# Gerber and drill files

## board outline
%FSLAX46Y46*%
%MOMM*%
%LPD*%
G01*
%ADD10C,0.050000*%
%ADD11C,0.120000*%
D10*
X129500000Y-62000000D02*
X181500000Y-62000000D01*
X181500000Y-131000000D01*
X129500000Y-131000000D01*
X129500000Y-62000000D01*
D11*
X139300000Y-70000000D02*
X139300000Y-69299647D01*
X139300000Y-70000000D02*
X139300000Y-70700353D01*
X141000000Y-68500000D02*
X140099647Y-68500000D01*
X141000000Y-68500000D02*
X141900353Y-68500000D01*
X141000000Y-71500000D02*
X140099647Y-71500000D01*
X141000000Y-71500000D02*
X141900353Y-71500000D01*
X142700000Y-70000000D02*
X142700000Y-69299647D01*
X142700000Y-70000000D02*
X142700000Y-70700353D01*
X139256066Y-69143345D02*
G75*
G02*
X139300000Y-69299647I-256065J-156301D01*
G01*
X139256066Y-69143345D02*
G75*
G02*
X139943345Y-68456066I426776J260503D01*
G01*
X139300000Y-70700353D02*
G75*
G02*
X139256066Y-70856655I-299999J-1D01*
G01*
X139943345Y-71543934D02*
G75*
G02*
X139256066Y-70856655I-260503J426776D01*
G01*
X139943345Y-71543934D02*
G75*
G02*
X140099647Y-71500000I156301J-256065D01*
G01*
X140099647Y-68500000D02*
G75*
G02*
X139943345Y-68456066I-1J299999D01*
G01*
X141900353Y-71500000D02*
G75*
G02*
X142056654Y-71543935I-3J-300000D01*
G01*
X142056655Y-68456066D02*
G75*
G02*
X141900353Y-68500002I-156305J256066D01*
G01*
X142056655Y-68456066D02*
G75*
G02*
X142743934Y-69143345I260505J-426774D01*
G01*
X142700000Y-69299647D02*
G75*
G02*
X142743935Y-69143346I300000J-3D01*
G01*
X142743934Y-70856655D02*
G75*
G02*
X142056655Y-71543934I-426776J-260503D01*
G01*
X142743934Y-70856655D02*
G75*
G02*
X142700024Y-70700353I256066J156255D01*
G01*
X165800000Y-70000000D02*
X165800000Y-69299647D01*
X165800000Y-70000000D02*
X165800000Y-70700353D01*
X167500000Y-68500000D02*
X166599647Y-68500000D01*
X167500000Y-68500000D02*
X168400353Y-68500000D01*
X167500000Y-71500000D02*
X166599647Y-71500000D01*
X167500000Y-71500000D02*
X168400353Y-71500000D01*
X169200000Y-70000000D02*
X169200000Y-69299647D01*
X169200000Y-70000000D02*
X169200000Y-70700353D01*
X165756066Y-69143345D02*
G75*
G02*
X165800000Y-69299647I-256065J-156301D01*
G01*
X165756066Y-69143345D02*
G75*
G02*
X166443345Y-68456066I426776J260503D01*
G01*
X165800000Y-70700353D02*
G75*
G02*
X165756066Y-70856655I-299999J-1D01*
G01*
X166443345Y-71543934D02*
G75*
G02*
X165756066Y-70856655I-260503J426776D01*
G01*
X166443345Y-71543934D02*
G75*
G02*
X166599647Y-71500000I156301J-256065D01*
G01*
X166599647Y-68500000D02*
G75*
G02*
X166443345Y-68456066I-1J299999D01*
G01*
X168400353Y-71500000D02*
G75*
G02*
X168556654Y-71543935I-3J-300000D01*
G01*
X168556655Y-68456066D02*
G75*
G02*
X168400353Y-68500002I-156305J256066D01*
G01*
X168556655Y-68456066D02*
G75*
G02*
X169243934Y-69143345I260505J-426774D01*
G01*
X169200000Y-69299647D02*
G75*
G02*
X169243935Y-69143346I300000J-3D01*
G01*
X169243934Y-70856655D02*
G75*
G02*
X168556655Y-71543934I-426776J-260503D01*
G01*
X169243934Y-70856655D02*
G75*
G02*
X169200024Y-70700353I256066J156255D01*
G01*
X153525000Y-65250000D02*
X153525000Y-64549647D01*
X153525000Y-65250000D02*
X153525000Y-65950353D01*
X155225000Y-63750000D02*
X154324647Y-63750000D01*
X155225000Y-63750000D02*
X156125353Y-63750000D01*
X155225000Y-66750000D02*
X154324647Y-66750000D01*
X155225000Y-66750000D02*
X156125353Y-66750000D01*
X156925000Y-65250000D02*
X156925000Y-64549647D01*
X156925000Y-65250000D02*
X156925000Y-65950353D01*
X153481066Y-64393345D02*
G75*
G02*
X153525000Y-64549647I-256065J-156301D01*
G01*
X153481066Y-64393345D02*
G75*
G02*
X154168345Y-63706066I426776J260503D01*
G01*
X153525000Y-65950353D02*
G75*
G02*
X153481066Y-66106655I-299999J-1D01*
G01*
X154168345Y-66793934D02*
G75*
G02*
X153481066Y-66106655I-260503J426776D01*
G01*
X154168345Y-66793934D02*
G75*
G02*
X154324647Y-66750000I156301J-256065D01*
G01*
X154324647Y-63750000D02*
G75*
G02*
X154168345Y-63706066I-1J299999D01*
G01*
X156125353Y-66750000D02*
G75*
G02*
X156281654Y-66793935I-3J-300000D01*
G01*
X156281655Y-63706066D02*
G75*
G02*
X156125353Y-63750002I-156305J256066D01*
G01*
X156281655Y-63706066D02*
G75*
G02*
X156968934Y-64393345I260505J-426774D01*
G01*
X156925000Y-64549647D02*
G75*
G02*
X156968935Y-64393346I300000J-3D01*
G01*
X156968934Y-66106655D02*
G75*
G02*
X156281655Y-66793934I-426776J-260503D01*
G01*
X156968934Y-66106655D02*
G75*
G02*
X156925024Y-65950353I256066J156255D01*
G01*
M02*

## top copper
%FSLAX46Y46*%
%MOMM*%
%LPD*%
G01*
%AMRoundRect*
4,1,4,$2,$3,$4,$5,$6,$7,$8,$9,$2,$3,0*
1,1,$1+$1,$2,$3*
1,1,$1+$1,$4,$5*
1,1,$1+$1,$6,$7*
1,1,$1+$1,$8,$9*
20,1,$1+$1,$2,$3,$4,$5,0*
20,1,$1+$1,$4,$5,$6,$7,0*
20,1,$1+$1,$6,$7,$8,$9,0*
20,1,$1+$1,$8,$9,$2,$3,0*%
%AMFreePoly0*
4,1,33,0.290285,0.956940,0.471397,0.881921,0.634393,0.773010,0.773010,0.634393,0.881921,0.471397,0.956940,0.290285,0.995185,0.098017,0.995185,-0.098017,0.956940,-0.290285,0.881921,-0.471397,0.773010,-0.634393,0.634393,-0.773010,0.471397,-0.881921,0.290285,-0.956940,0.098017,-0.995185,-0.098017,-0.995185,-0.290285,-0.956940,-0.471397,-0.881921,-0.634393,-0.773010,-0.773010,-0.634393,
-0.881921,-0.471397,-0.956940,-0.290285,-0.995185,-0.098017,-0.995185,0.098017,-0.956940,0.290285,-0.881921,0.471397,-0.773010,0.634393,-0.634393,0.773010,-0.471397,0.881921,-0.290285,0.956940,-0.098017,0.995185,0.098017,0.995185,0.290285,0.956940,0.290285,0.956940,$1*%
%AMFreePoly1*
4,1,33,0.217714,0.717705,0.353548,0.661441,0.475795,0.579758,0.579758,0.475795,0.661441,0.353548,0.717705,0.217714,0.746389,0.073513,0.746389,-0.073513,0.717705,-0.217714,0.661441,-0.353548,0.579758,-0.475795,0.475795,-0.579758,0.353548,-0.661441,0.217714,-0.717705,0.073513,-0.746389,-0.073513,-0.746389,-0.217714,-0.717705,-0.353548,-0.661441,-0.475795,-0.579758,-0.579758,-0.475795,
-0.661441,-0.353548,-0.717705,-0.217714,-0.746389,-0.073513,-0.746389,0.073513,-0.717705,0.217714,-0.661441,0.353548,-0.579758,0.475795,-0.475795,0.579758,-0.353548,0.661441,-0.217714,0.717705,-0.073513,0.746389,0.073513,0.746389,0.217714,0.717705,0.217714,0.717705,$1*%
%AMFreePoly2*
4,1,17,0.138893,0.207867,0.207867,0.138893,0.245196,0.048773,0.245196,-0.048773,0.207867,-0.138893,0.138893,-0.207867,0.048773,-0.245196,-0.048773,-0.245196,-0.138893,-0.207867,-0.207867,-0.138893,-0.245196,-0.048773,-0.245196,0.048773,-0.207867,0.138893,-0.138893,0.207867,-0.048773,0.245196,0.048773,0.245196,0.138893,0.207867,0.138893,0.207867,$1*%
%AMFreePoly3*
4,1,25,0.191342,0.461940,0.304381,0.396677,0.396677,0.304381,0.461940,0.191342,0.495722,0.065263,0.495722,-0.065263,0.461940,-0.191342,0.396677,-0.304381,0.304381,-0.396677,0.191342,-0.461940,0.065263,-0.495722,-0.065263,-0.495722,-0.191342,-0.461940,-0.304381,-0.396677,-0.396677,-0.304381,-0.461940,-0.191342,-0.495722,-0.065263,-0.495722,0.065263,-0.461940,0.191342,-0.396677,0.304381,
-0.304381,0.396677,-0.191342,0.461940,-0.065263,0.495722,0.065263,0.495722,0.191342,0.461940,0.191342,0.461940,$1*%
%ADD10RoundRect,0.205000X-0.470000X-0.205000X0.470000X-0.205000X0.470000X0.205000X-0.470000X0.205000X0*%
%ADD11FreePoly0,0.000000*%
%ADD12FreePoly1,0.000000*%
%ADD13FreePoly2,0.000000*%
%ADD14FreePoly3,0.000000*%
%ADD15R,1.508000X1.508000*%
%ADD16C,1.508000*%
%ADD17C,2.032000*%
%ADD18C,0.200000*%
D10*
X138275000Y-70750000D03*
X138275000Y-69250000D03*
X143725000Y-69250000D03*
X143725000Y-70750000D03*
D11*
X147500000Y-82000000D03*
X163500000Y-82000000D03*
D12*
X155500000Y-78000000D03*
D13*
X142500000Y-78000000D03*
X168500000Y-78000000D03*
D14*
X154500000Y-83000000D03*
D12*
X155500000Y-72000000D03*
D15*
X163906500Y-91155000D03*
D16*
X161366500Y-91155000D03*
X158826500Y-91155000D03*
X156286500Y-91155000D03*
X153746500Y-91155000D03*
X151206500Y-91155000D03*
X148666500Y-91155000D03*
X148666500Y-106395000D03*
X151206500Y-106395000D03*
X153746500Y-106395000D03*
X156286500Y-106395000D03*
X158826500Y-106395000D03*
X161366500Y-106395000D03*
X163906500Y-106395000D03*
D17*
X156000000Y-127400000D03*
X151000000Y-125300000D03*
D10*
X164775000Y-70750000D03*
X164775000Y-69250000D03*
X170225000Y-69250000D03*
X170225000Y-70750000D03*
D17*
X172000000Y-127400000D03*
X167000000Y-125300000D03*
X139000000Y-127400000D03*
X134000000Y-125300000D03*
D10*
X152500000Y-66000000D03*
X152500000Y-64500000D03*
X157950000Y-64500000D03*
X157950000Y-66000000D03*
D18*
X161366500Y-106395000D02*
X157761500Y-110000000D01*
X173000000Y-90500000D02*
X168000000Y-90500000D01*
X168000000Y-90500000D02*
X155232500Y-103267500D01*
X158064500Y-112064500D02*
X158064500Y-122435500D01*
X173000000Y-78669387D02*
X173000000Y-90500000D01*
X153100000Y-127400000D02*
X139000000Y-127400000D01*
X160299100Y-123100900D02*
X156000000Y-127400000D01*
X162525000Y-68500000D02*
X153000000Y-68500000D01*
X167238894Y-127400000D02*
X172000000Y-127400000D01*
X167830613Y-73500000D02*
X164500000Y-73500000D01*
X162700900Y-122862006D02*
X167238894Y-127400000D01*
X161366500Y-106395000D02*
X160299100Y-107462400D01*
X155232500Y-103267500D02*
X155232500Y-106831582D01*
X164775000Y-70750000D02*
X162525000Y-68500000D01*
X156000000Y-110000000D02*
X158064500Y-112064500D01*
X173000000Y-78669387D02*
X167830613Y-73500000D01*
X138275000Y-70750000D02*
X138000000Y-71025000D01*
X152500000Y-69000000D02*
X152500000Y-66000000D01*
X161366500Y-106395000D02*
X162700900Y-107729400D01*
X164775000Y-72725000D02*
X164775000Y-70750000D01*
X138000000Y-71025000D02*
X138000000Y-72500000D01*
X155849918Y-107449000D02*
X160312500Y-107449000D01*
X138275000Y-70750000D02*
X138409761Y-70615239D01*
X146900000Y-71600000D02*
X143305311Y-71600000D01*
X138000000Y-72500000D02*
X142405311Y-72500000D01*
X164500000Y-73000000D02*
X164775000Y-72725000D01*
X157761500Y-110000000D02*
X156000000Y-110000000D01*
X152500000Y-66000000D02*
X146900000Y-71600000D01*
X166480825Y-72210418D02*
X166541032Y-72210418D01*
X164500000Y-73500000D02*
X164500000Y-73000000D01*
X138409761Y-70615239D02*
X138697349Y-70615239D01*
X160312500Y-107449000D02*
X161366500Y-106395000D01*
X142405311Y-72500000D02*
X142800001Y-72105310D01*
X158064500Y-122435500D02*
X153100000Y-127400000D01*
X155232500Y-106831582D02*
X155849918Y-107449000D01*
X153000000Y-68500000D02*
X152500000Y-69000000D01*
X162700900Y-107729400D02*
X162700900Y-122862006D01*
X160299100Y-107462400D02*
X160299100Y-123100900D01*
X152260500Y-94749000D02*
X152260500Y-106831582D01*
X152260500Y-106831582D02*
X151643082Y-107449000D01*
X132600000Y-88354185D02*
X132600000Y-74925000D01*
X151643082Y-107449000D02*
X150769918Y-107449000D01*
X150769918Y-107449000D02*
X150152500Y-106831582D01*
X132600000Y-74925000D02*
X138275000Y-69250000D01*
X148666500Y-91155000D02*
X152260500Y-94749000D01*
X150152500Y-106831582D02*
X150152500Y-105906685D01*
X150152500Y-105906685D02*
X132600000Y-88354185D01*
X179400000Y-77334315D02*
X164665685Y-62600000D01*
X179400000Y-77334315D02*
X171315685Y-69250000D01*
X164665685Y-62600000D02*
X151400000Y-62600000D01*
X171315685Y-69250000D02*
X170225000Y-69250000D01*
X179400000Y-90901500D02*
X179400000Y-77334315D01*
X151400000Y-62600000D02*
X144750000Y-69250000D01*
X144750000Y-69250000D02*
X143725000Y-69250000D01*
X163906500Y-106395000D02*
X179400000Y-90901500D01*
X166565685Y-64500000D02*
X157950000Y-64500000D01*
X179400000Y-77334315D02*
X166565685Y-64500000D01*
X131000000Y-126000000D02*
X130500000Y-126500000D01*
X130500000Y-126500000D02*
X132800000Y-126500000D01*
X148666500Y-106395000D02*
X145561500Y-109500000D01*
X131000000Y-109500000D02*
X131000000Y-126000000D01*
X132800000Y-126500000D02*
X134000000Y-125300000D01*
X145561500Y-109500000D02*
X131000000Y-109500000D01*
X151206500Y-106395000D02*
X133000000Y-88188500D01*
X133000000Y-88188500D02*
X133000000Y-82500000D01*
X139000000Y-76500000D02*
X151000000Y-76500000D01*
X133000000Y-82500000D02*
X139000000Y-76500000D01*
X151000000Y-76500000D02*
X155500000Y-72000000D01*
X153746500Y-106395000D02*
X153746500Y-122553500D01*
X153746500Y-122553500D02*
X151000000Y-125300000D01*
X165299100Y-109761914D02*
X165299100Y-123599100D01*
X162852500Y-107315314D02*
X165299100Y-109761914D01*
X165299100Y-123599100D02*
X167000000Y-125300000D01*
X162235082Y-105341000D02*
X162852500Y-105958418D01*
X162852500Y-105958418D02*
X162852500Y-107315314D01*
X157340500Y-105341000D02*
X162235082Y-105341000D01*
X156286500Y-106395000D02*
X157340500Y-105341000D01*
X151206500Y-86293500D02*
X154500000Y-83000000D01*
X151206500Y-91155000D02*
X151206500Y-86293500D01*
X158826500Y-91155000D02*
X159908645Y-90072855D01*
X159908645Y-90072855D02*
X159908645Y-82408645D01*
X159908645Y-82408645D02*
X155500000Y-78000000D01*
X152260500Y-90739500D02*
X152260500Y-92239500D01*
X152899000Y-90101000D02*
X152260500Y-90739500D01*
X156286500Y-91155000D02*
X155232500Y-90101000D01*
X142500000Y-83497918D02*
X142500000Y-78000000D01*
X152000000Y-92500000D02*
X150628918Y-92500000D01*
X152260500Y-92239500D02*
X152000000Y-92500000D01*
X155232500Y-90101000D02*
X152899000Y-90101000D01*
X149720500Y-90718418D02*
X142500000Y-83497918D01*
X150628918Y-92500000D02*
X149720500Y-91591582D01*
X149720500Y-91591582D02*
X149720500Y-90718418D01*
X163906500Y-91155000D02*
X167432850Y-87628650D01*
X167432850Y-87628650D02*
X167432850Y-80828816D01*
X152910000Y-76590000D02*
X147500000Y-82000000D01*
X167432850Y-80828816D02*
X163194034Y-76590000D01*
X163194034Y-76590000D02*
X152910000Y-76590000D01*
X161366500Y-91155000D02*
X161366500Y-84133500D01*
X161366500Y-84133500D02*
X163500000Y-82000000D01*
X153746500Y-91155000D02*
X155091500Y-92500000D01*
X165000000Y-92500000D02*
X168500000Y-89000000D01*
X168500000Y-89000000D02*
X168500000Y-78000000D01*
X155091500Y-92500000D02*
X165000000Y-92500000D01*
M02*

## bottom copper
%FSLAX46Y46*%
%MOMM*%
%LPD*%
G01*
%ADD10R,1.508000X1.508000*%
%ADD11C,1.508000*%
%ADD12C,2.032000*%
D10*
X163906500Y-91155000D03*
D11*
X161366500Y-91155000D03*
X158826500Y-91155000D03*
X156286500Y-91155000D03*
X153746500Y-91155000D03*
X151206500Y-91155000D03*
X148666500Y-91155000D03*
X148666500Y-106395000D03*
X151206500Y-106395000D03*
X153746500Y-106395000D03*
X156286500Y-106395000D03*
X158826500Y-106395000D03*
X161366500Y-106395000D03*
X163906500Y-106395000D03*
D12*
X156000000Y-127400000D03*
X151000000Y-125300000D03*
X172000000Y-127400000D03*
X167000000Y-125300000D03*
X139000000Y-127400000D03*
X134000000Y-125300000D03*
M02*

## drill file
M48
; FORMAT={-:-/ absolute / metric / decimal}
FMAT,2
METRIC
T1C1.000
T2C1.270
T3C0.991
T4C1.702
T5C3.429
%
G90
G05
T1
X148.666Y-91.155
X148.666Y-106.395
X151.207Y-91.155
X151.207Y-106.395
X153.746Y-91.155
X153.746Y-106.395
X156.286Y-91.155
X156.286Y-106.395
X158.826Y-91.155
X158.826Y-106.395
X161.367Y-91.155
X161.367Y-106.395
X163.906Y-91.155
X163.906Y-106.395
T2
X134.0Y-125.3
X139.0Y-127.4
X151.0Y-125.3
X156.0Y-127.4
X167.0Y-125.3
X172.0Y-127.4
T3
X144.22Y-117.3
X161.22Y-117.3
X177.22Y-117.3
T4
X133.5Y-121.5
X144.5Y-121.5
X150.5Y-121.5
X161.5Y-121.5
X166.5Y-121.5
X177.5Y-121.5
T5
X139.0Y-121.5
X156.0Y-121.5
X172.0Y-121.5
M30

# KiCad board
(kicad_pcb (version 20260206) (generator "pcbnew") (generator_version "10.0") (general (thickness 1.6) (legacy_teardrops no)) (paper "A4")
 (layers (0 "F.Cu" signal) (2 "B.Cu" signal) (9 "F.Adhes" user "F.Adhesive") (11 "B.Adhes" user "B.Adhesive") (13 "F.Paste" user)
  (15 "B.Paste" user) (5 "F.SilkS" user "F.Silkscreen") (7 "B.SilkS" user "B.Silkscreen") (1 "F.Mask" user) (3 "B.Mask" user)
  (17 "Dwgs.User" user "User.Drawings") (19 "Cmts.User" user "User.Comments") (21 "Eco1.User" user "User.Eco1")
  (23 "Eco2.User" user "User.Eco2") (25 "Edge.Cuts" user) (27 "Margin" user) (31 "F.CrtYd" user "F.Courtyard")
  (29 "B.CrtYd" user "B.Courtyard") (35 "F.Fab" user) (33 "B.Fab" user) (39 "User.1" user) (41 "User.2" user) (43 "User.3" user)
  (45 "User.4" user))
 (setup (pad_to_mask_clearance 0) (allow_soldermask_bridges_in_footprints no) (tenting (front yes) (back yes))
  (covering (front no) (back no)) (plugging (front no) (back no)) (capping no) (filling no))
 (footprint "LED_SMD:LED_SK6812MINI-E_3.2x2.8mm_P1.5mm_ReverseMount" (layer "F.Cu") (at 141 70)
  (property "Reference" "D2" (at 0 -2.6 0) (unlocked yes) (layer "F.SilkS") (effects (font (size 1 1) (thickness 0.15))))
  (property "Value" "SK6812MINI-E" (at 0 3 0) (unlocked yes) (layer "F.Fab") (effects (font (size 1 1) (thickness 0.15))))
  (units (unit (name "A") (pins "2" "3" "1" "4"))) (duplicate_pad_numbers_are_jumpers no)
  (fp_line (start -1.7 0) (end -1.7 -0.700353) (stroke (width 0.12) (type solid)) (layer "Edge.Cuts"))
  (fp_line (start -1.7 0) (end -1.7 0.700353) (stroke (width 0.12) (type solid)) (layer "Edge.Cuts"))
  (fp_line (start 0 -1.5) (end -0.900353 -1.5) (stroke (width 0.12) (type solid)) (layer "Edge.Cuts"))
  (fp_line (start 0 -1.5) (end 0.900353 -1.5) (stroke (width 0.12) (type solid)) (layer "Edge.Cuts"))
  (fp_line (start 0 1.5) (end -0.900353 1.5) (stroke (width 0.12) (type solid)) (layer "Edge.Cuts"))
  (fp_line (start 0 1.5) (end 0.900353 1.5) (stroke (width 0.12) (type solid)) (layer "Edge.Cuts"))
  (fp_line (start 1.7 0) (end 1.7 -0.700353) (stroke (width 0.12) (type solid)) (layer "Edge.Cuts"))
  (fp_line (start 1.7 0) (end 1.7 0.700353) (stroke (width 0.12) (type solid)) (layer "Edge.Cuts"))
  (fp_arc (start -1.743934 -0.856655) (mid -1.711192 -0.781532) (end -1.7 -0.700353) (stroke (width 0.12) (type solid)) (layer "Edge.Cuts"))
  (fp_arc (start -1.743934 -0.856655) (mid -1.670711 -1.470711) (end -1.056655 -1.543934) (stroke (width 0.12) (type solid))
   (layer "Edge.Cuts"))
  (fp_arc (start -1.7 0.700353) (mid -1.711192 0.781532) (end -1.743934 0.856655) (stroke (width 0.12) (type solid)) (layer "Edge.Cuts"))
  (fp_arc (start -1.056655 1.543934) (mid -1.670711 1.470711) (end -1.743934 0.856655) (stroke (width 0.12) (type solid))
   (layer "Edge.Cuts"))
  (fp_arc (start -1.056655 1.543934) (mid -0.981532 1.511192) (end -0.900353 1.5) (stroke (width 0.12) (type solid)) (layer "Edge.Cuts"))
  (fp_arc (start -0.900353 -1.5) (mid -0.981532 -1.511192) (end -1.056655 -1.543934) (stroke (width 0.12) (type solid)) (layer "Edge.Cuts"))
  (fp_arc (start 0.900353 1.5) (mid 0.981532 1.511192) (end 1.056655 1.543934) (stroke (width 0.12) (type solid)) (layer "Edge.Cuts"))
  (fp_arc (start 1.056655 -1.543934) (mid 0.981532 -1.511192) (end 0.900353 -1.5) (stroke (width 0.12) (type solid)) (layer "Edge.Cuts"))
  (fp_arc (start 1.056655 -1.543934) (mid 1.670711 -1.470711) (end 1.743934 -0.856655) (stroke (width 0.12) (type solid))
   (layer "Edge.Cuts"))
  (fp_arc (start 1.7 -0.700353) (mid 1.711192 -0.781532) (end 1.743934 -0.856655) (stroke (width 0.12) (type solid)) (layer "Edge.Cuts"))
  (fp_arc (start 1.743934 0.856655) (mid 1.670711 1.470711) (end 1.056655 1.543934) (stroke (width 0.12) (type solid)) (layer "Edge.Cuts"))
  (fp_arc (start 1.743934 0.856655) (mid 1.711192 0.781532) (end 1.7 0.700353) (stroke (width 0.12) (type solid)) (layer "Edge.Cuts"))
  (pad "1" smd roundrect (at -2.725 0.75) (size 1.35 0.82) (layers "F.Cu" "F.Mask" "F.Paste") (roundrect_rratio 0.25) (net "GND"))
  (pad "2" smd roundrect (at -2.725 -0.75) (size 1.35 0.82) (layers "F.Cu" "F.Mask" "F.Paste") (roundrect_rratio 0.25) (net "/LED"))
  (pad "3" smd roundrect (at 2.725 -0.75) (size 1.35 0.82) (layers "F.Cu" "F.Mask" "F.Paste") (roundrect_rratio 0.25) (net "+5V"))
  (pad "4" smd roundrect (at 2.725 0.75) (size 1.35 0.82) (layers "F.Cu" "F.Mask" "F.Paste") (roundrect_rratio 0.25) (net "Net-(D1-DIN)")))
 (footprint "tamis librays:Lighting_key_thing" (layer "F.Cu") (at 149.5 71)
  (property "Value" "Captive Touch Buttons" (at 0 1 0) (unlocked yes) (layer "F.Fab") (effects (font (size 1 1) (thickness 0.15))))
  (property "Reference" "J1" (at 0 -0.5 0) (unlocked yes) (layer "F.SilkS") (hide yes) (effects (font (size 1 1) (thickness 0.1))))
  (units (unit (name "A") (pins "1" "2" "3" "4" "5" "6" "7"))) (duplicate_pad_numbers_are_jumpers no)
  (pad "1" smd custom (at -2 11) (size 2 2) (layers "F.Cu" "F.Mask") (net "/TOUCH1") (thermal_bridge_angle 90)
   (options (clearance outline) (anchor circle)) (primitives))
  (pad "2" smd custom (at 14 11) (size 2 2) (layers "F.Cu" "F.Mask") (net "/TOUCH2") (thermal_bridge_angle 90)
   (options (clearance outline) (anchor circle)) (primitives))
  (pad "3" smd custom (at 6 7) (size 1.5 5) (layers "F.Cu" "F.Mask") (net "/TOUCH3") (thermal_bridge_angle 90)
   (options (clearance outline) (anchor circle)) (primitives))
  (pad "4" smd custom (at -7 7) (size 0.5 0.5) (layers "F.Cu" "F.Mask") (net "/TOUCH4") (thermal_bridge_angle 90)
   (options (clearance outline) (anchor circle)) (primitives))
  (pad "5" smd custom (at 19 7) (size 0.5 0.5) (layers "F.Cu" "F.Mask") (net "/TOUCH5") (thermal_bridge_angle 90)
   (options (clearance outline) (anchor circle)) (primitives))
  (pad "6" smd custom (at 5 12) (size 1 1) (layers "F.Cu" "F.Mask") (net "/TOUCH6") (thermal_bridge_angle 90)
   (options (clearance outline) (anchor circle)) (primitives))
  (pad "7" smd custom (at 6 1) (size 1.5 1.5) (layers "F.Cu" "F.Mask") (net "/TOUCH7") (thermal_bridge_angle 90)
   (options (clearance outline) (anchor circle)) (primitives)))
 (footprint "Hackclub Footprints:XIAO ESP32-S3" (layer "F.Cu") (at 156.35 98.775 -90)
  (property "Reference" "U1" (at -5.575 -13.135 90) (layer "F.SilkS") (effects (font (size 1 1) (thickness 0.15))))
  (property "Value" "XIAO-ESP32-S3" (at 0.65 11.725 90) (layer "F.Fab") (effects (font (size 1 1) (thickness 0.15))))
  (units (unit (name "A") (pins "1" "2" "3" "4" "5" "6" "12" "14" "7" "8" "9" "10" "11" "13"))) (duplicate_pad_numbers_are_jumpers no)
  (pad "1" thru_hole rect (at -7.62 -7.5565 270) (size 1.508 1.508) (drill 1) (layers "*.Cu" "*.Mask") (remove_unused_layers no)
   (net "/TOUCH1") (solder_mask_margin 0.102))
  (pad "2" thru_hole circle (at -7.62 -5.0165 270) (size 1.508 1.508) (drill 1) (layers "*.Cu" "*.Mask") (remove_unused_layers no)
   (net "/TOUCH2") (solder_mask_margin 0.102))
  (pad "3" thru_hole circle (at -7.62 -2.4765 270) (size 1.508 1.508) (drill 1) (layers "*.Cu" "*.Mask") (remove_unused_layers no)
   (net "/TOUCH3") (solder_mask_margin 0.102))
  (pad "4" thru_hole circle (at -7.62 0.0635 270) (size 1.508 1.508) (drill 1) (layers "*.Cu" "*.Mask") (remove_unused_layers no)
   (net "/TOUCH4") (solder_mask_margin 0.102))
  (pad "5" thru_hole circle (at -7.62 2.6035 270) (size 1.508 1.508) (drill 1) (layers "*.Cu" "*.Mask") (remove_unused_layers no)
   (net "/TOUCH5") (solder_mask_margin 0.102))
  (pad "6" thru_hole circle (at -7.62 5.1435 270) (size 1.508 1.508) (drill 1) (layers "*.Cu" "*.Mask") (remove_unused_layers no)
   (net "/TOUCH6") (solder_mask_margin 0.102))
  (pad "7" thru_hole circle (at -7.62 7.6835 270) (size 1.508 1.508) (drill 1) (layers "*.Cu" "*.Mask") (remove_unused_layers no)
   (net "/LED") (solder_mask_margin 0.102))
  (pad "8" thru_hole circle (at 7.62 7.6835 270) (size 1.508 1.508) (drill 1) (layers "*.Cu" "*.Mask") (remove_unused_layers no)
   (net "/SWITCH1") (solder_mask_margin 0.102))
  (pad "9" thru_hole circle (at 7.62 5.1435 270) (size 1.508 1.508) (drill 1) (layers "*.Cu" "*.Mask") (remove_unused_layers no)
   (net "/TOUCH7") (solder_mask_margin 0.102))
  (pad "10" thru_hole circle (at 7.62 2.6035 270) (size 1.508 1.508) (drill 1) (layers "*.Cu" "*.Mask") (remove_unused_layers no)
   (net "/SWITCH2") (solder_mask_margin 0.102))
  (pad "11" thru_hole circle (at 7.62 0.0635 270) (size 1.508 1.508) (drill 1) (layers "*.Cu" "*.Mask") (remove_unused_layers no)
   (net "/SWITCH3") (solder_mask_margin 0.102))
  (pad "12" thru_hole circle (at 7.62 -2.4765 270) (size 1.508 1.508) (drill 1) (layers "*.Cu" "*.Mask") (remove_unused_layers no)
   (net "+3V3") (solder_mask_margin 0.102))
  (pad "13" thru_hole circle (at 7.62 -5.0165 270) (size 1.508 1.508) (drill 1) (layers "*.Cu" "*.Mask") (remove_unused_layers no)
   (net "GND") (solder_mask_margin 0.102))
  (pad "14" thru_hole circle (at 7.62 -7.5565 270) (size 1.508 1.508) (drill 1) (layers "*.Cu" "*.Mask") (remove_unused_layers no)
   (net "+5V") (solder_mask_margin 0.102)))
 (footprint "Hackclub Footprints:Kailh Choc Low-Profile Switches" (layer "F.Cu") (at 156 121.5)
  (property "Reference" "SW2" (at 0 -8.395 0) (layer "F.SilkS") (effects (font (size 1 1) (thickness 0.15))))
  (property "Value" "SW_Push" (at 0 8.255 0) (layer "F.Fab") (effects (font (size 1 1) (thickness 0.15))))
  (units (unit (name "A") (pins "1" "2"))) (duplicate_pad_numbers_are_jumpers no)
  (pad "" np_thru_hole circle (at -5.5 0) (size 1.7018 1.7018) (drill 1.7018) (layers "*.Cu" "*.Mask"))
  (pad "" np_thru_hole circle (at 0 0) (size 3.429 3.429) (drill 3.429) (layers "*.Cu" "*.Mask"))
  (pad "" np_thru_hole circle (at 5.22 -4.2) (size 0.9906 0.9906) (drill 0.9906) (layers "*.Cu" "*.Mask"))
  (pad "" np_thru_hole circle (at 5.5 0) (size 1.7018 1.7018) (drill 1.7018) (layers "*.Cu" "*.Mask"))
  (pad "1" thru_hole circle (at 0 5.9) (size 2.032 2.032) (drill 1.27) (layers "*.Cu" "*.Mask") (remove_unused_layers no) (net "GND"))
  (pad "2" thru_hole circle (at -5 3.8) (size 2.032 2.032) (drill 1.27) (layers "*.Cu" "*.Mask") (remove_unused_layers no) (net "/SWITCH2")))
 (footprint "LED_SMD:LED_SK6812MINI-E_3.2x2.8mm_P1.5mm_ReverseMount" (layer "F.Cu") (at 167.5 70)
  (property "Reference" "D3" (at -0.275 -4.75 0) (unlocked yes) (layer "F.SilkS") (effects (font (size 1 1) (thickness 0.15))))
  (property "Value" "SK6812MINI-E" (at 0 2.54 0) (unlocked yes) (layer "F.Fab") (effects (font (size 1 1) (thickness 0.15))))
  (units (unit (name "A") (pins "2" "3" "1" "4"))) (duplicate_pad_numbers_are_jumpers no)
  (fp_line (start -1.7 0) (end -1.7 -0.700353) (stroke (width 0.12) (type solid)) (layer "Edge.Cuts"))
  (fp_line (start -1.7 0) (end -1.7 0.700353) (stroke (width 0.12) (type solid)) (layer "Edge.Cuts"))
  (fp_line (start 0 -1.5) (end -0.900353 -1.5) (stroke (width 0.12) (type solid)) (layer "Edge.Cuts"))
  (fp_line (start 0 -1.5) (end 0.900353 -1.5) (stroke (width 0.12) (type solid)) (layer "Edge.Cuts"))
  (fp_line (start 0 1.5) (end -0.900353 1.5) (stroke (width 0.12) (type solid)) (layer "Edge.Cuts"))
  (fp_line (start 0 1.5) (end 0.900353 1.5) (stroke (width 0.12) (type solid)) (layer "Edge.Cuts"))
  (fp_line (start 1.7 0) (end 1.7 -0.700353) (stroke (width 0.12) (type solid)) (layer "Edge.Cuts"))
  (fp_line (start 1.7 0) (end 1.7 0.700353) (stroke (width 0.12) (type solid)) (layer "Edge.Cuts"))
  (fp_arc (start -1.743934 -0.856655) (mid -1.711192 -0.781532) (end -1.7 -0.700353) (stroke (width 0.12) (type solid)) (layer "Edge.Cuts"))
  (fp_arc (start -1.743934 -0.856655) (mid -1.670711 -1.470711) (end -1.056655 -1.543934) (stroke (width 0.12) (type solid))
   (layer "Edge.Cuts"))
  (fp_arc (start -1.7 0.700353) (mid -1.711192 0.781532) (end -1.743934 0.856655) (stroke (width 0.12) (type solid)) (layer "Edge.Cuts"))
  (fp_arc (start -1.056655 1.543934) (mid -1.670711 1.470711) (end -1.743934 0.856655) (stroke (width 0.12) (type solid))
   (layer "Edge.Cuts"))
  (fp_arc (start -1.056655 1.543934) (mid -0.981532 1.511192) (end -0.900353 1.5) (stroke (width 0.12) (type solid)) (layer "Edge.Cuts"))
  (fp_arc (start -0.900353 -1.5) (mid -0.981532 -1.511192) (end -1.056655 -1.543934) (stroke (width 0.12) (type solid)) (layer "Edge.Cuts"))
  (fp_arc (start 0.900353 1.5) (mid 0.981532 1.511192) (end 1.056655 1.543934) (stroke (width 0.12) (type solid)) (layer "Edge.Cuts"))
  (fp_arc (start 1.056655 -1.543934) (mid 0.981532 -1.511192) (end 0.900353 -1.5) (stroke (width 0.12) (type solid)) (layer "Edge.Cuts"))
  (fp_arc (start 1.056655 -1.543934) (mid 1.670711 -1.470711) (end 1.743934 -0.856655) (stroke (width 0.12) (type solid))
   (layer "Edge.Cuts"))
  (fp_arc (start 1.7 -0.700353) (mid 1.711192 -0.781532) (end 1.743934 -0.856655) (stroke (width 0.12) (type solid)) (layer "Edge.Cuts"))
  (fp_arc (start 1.743934 0.856655) (mid 1.670711 1.470711) (end 1.056655 1.543934) (stroke (width 0.12) (type solid)) (layer "Edge.Cuts"))
  (fp_arc (start 1.743934 0.856655) (mid 1.711192 0.781532) (end 1.7 0.700353) (stroke (width 0.12) (type solid)) (layer "Edge.Cuts"))
  (pad "1" smd roundrect (at -2.725 0.75) (size 1.35 0.82) (layers "F.Cu" "F.Mask" "F.Paste") (roundrect_rratio 0.25) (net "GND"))
  (pad "2" smd roundrect (at -2.725 -0.75) (size 1.35 0.82) (layers "F.Cu" "F.Mask" "F.Paste") (roundrect_rratio 0.25) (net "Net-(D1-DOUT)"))
  (pad "3" smd roundrect (at 2.725 -0.75) (size 1.35 0.82) (layers "F.Cu" "F.Mask" "F.Paste") (roundrect_rratio 0.25) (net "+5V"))
  (pad "4" smd roundrect (at 2.725 0.75) (size 1.35 0.82) (layers "F.Cu" "F.Mask" "F.Paste") (roundrect_rratio 0.25)
   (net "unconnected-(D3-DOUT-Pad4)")))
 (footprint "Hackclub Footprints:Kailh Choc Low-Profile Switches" (layer "F.Cu") (at 172 121.5)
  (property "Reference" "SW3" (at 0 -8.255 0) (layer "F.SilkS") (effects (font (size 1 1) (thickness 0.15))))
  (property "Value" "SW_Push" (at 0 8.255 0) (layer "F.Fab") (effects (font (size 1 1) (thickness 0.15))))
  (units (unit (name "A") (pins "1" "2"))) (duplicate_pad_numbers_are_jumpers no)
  (pad "" np_thru_hole circle (at -5.5 0) (size 1.7018 1.7018) (drill 1.7018) (layers "*.Cu" "*.Mask"))
  (pad "" np_thru_hole circle (at 0 0) (size 3.429 3.429) (drill 3.429) (layers "*.Cu" "*.Mask"))
  (pad "" np_thru_hole circle (at 5.22 -4.2) (size 0.9906 0.9906) (drill 0.9906) (layers "*.Cu" "*.Mask"))
  (pad "" np_thru_hole circle (at 5.5 0) (size 1.7018 1.7018) (drill 1.7018) (layers "*.Cu" "*.Mask"))
  (pad "1" thru_hole circle (at 0 5.9) (size 2.032 2.032) (drill 1.27) (layers "*.Cu" "*.Mask") (remove_unused_layers no) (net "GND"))
  (pad "2" thru_hole circle (at -5 3.8) (size 2.032 2.032) (drill 1.27) (layers "*.Cu" "*.Mask") (remove_unused_layers no) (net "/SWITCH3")))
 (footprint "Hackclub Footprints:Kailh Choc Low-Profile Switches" (layer "F.Cu") (at 139 121.5)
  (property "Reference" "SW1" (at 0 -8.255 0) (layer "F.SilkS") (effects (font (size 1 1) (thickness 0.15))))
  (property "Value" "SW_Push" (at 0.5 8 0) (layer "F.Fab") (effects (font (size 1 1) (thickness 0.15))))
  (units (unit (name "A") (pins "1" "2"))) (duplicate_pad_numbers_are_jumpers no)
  (pad "" np_thru_hole circle (at -5.5 0) (size 1.7018 1.7018) (drill 1.7018) (layers "*.Cu" "*.Mask"))
  (pad "" np_thru_hole circle (at 0 0) (size 3.429 3.429) (drill 3.429) (layers "*.Cu" "*.Mask"))
  (pad "" np_thru_hole circle (at 5.22 -4.2) (size 0.9906 0.9906) (drill 0.9906) (layers "*.Cu" "*.Mask"))
  (pad "" np_thru_hole circle (at 5.5 0) (size 1.7018 1.7018) (drill 1.7018) (layers "*.Cu" "*.Mask"))
  (pad "1" thru_hole circle (at 0 5.9) (size 2.032 2.032) (drill 1.27) (layers "*.Cu" "*.Mask") (remove_unused_layers no) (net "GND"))
  (pad "2" thru_hole circle (at -5 3.8) (size 2.032 2.032) (drill 1.27) (layers "*.Cu" "*.Mask") (remove_unused_layers no) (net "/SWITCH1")))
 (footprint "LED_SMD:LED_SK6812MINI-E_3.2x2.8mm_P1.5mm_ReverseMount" (layer "F.Cu") (at 155.225 65.25)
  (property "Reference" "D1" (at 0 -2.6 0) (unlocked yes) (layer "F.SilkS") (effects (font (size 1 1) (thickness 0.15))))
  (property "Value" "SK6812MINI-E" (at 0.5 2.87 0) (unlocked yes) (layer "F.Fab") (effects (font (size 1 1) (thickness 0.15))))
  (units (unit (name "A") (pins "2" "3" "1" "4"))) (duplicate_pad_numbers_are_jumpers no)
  (fp_line (start -1.7 0) (end -1.7 -0.700353) (stroke (width 0.12) (type solid)) (layer "Edge.Cuts"))
  (fp_line (start -1.7 0) (end -1.7 0.700353) (stroke (width 0.12) (type solid)) (layer "Edge.Cuts"))
  (fp_line (start 0 -1.5) (end -0.900353 -1.5) (stroke (width 0.12) (type solid)) (layer "Edge.Cuts"))
  (fp_line (start 0 -1.5) (end 0.900353 -1.5) (stroke (width 0.12) (type solid)) (layer "Edge.Cuts"))
  (fp_line (start 0 1.5) (end -0.900353 1.5) (stroke (width 0.12) (type solid)) (layer "Edge.Cuts"))
  (fp_line (start 0 1.5) (end 0.900353 1.5) (stroke (width 0.12) (type solid)) (layer "Edge.Cuts"))
  (fp_line (start 1.7 0) (end 1.7 -0.700353) (stroke (width 0.12) (type solid)) (layer "Edge.Cuts"))
  (fp_line (start 1.7 0) (end 1.7 0.700353) (stroke (width 0.12) (type solid)) (layer "Edge.Cuts"))
  (fp_arc (start -1.743934 -0.856655) (mid -1.711192 -0.781532) (end -1.7 -0.700353) (stroke (width 0.12) (type solid)) (layer "Edge.Cuts"))
  (fp_arc (start -1.743934 -0.856655) (mid -1.670711 -1.470711) (end -1.056655 -1.543934) (stroke (width 0.12) (type solid))
   (layer "Edge.Cuts"))
  (fp_arc (start -1.7 0.700353) (mid -1.711192 0.781532) (end -1.743934 0.856655) (stroke (width 0.12) (type solid)) (layer "Edge.Cuts"))
  (fp_arc (start -1.056655 1.543934) (mid -1.670711 1.470711) (end -1.743934 0.856655) (stroke (width 0.12) (type solid))
   (layer "Edge.Cuts"))
  (fp_arc (start -1.056655 1.543934) (mid -0.981532 1.511192) (end -0.900353 1.5) (stroke (width 0.12) (type solid)) (layer "Edge.Cuts"))
  (fp_arc (start -0.900353 -1.5) (mid -0.981532 -1.511192) (end -1.056655 -1.543934) (stroke (width 0.12) (type solid)) (layer "Edge.Cuts"))
  (fp_arc (start 0.900353 1.5) (mid 0.981532 1.511192) (end 1.056655 1.543934) (stroke (width 0.12) (type solid)) (layer "Edge.Cuts"))
  (fp_arc (start 1.056655 -1.543934) (mid 0.981532 -1.511192) (end 0.900353 -1.5) (stroke (width 0.12) (type solid)) (layer "Edge.Cuts"))
  (fp_arc (start 1.056655 -1.543934) (mid 1.670711 -1.470711) (end 1.743934 -0.856655) (stroke (width 0.12) (type solid))
   (layer "Edge.Cuts"))
  (fp_arc (start 1.7 -0.700353) (mid 1.711192 -0.781532) (end 1.743934 -0.856655) (stroke (width 0.12) (type solid)) (layer "Edge.Cuts"))
  (fp_arc (start 1.743934 0.856655) (mid 1.670711 1.470711) (end 1.056655 1.543934) (stroke (width 0.12) (type solid)) (layer "Edge.Cuts"))
  (fp_arc (start 1.743934 0.856655) (mid 1.711192 0.781532) (end 1.7 0.700353) (stroke (width 0.12) (type solid)) (layer "Edge.Cuts"))
  (pad "1" smd roundrect (at -2.725 0.75) (size 1.35 0.82) (layers "F.Cu" "F.Mask" "F.Paste") (roundrect_rratio 0.25) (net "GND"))
  (pad "2" smd roundrect (at -2.725 -0.75) (size 1.35 0.82) (layers "F.Cu" "F.Mask" "F.Paste") (roundrect_rratio 0.25) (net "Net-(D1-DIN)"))
  (pad "3" smd roundrect (at 2.725 -0.75) (size 1.35 0.82) (layers "F.Cu" "F.Mask" "F.Paste") (roundrect_rratio 0.25) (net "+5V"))
  (pad "4" smd roundrect (at 2.725 0.75) (size 1.35 0.82) (layers "F.Cu" "F.Mask" "F.Paste") (roundrect_rratio 0.25) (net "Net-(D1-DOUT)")))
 (gr_rect (start 129.5 62) (end 181.5 131) (stroke (width 0.05) (type default)) (fill no) (layer "Edge.Cuts"))
 (segment (start 161.3665 106.395) (end 157.7615 110) (width 0.2) (layer "F.Cu") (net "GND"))
 (segment (start 173 90.5) (end 168 90.5) (width 0.2) (layer "F.Cu") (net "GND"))
 (segment (start 168 90.5) (end 155.2325 103.2675) (width 0.2) (layer "F.Cu") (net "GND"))
 (segment (start 158.0645 112.0645) (end 158.0645 122.4355) (width 0.2) (layer "F.Cu") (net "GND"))
 (segment (start 173 78.669387) (end 173 90.5) (width 0.2) (layer "F.Cu") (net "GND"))
 (segment (start 153.1 127.4) (end 139 127.4) (width 0.2) (layer "F.Cu") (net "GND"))
 (segment (start 160.2991 123.1009) (end 156 127.4) (width 0.2) (layer "F.Cu") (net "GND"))
 (segment (start 162.525 68.5) (end 153 68.5) (width 0.2) (layer "F.Cu") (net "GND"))
 (segment (start 167.238894 127.4) (end 172 127.4) (width 0.2) (layer "F.Cu") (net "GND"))
 (segment (start 167.830613 73.5) (end 164.5 73.5) (width 0.2) (layer "F.Cu") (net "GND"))
 (segment (start 162.7009 122.862006) (end 167.238894 127.4) (width 0.2) (layer "F.Cu") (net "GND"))
 (segment (start 161.3665 106.395) (end 160.2991 107.4624) (width 0.2) (layer "F.Cu") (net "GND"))
 (segment (start 155.2325 103.2675) (end 155.2325 106.831582) (width 0.2) (layer "F.Cu") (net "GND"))
 (segment (start 164.775 70.75) (end 162.525 68.5) (width 0.2) (layer "F.Cu") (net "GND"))
 (segment (start 156 110) (end 158.0645 112.0645) (width 0.2) (layer "F.Cu") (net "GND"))
 (segment (start 173 78.669387) (end 167.830613 73.5) (width 0.2) (layer "F.Cu") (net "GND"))
 (segment (start 138.275 70.75) (end 138 71.025) (width 0.2) (layer "F.Cu") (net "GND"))
 (segment (start 152.5 69) (end 152.5 66) (width 0.2) (layer "F.Cu") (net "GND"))
 (segment (start 161.3665 106.395) (end 162.7009 107.7294) (width 0.2) (layer "F.Cu") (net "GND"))
 (segment (start 164.775 72.725) (end 164.775 70.75) (width 0.2) (layer "F.Cu") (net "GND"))
 (segment (start 138 71.025) (end 138 72.5) (width 0.2) (layer "F.Cu") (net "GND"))
 (segment (start 155.849918 107.449) (end 160.3125 107.449) (width 0.2) (layer "F.Cu") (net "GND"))
 (segment (start 138.275 70.75) (end 138.409761 70.615239) (width 0.2) (layer "F.Cu") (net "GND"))
 (segment (start 146.9 71.6) (end 143.305311 71.6) (width 0.2) (layer "F.Cu") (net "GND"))
 (segment (start 138 72.5) (end 142.405311 72.5) (width 0.2) (layer "F.Cu") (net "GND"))
 (segment (start 164.5 73) (end 164.775 72.725) (width 0.2) (layer "F.Cu") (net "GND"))
 (segment (start 157.7615 110) (end 156 110) (width 0.2) (layer "F.Cu") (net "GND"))
 (segment (start 152.5 66) (end 146.9 71.6) (width 0.2) (layer "F.Cu") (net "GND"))
 (segment (start 166.480825 72.210418) (end 166.541032 72.210418) (width 0.2) (layer "F.Cu") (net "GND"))
 (segment (start 164.5 73.5) (end 164.5 73) (width 0.2) (layer "F.Cu") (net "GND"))
 (segment (start 138.409761 70.615239) (end 138.697349 70.615239) (width 0.2) (layer "F.Cu") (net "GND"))
 (segment (start 160.3125 107.449) (end 161.3665 106.395) (width 0.2) (layer "F.Cu") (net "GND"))
 (segment (start 142.405311 72.5) (end 142.800001 72.10531) (width 0.2) (layer "F.Cu") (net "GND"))
 (segment (start 158.0645 122.4355) (end 153.1 127.4) (width 0.2) (layer "F.Cu") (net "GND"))
 (segment (start 155.2325 106.831582) (end 155.849918 107.449) (width 0.2) (layer "F.Cu") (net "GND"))
 (segment (start 153 68.5) (end 152.5 69) (width 0.2) (layer "F.Cu") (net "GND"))
 (segment (start 162.7009 107.7294) (end 162.7009 122.862006) (width 0.2) (layer "F.Cu") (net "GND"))
 (segment (start 160.2991 107.4624) (end 160.2991 123.1009) (width 0.2) (layer "F.Cu") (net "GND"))
 (segment (start 152.2605 94.749) (end 152.2605 106.831582) (width 0.2) (layer "F.Cu") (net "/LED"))
 (segment (start 152.2605 106.831582) (end 151.643082 107.449) (width 0.2) (layer "F.Cu") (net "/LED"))
 (segment (start 132.6 88.354185) (end 132.6 74.925) (width 0.2) (layer "F.Cu") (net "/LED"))
 (segment (start 151.643082 107.449) (end 150.769918 107.449) (width 0.2) (layer "F.Cu") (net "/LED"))
 (segment (start 150.769918 107.449) (end 150.1525 106.831582) (width 0.2) (layer "F.Cu") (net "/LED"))
 (segment (start 132.6 74.925) (end 138.275 69.25) (width 0.2) (layer "F.Cu") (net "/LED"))
 (segment (start 148.6665 91.155) (end 152.2605 94.749) (width 0.2) (layer "F.Cu") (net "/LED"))
 (segment (start 150.1525 106.831582) (end 150.1525 105.906685) (width 0.2) (layer "F.Cu") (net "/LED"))
 (segment (start 150.1525 105.906685) (end 132.6 88.354185) (width 0.2) (layer "F.Cu") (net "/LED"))
 (segment (start 179.4 77.334315) (end 164.665685 62.6) (width 0.2) (layer "F.Cu") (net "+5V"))
 (segment (start 179.4 77.334315) (end 171.315685 69.25) (width 0.2) (layer "F.Cu") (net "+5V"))
 (segment (start 164.665685 62.6) (end 151.4 62.6) (width 0.2) (layer "F.Cu") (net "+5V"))
 (segment (start 171.315685 69.25) (end 170.225 69.25) (width 0.2) (layer "F.Cu") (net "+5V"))
 (segment (start 179.4 90.9015) (end 179.4 77.334315) (width 0.2) (layer "F.Cu") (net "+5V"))
 (segment (start 151.4 62.6) (end 144.75 69.25) (width 0.2) (layer "F.Cu") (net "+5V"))
 (segment (start 144.75 69.25) (end 143.725 69.25) (width 0.2) (layer "F.Cu") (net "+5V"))
 (segment (start 163.9065 106.395) (end 179.4 90.9015) (width 0.2) (layer "F.Cu") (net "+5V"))
 (segment (start 166.565685 64.5) (end 157.95 64.5) (width 0.2) (layer "F.Cu") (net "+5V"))
 (segment (start 179.4 77.334315) (end 166.565685 64.5) (width 0.2) (layer "F.Cu") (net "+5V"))
 (segment (start 131 126) (end 130.5 126.5) (width 0.2) (layer "F.Cu") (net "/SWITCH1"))
 (segment (start 130.5 126.5) (end 132.8 126.5) (width 0.2) (layer "F.Cu") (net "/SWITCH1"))
 (segment (start 148.6665 106.395) (end 145.5615 109.5) (width 0.2) (layer "F.Cu") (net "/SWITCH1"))
 (segment (start 131 109.5) (end 131 126) (width 0.2) (layer "F.Cu") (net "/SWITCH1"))
 (segment (start 132.8 126.5) (end 134 125.3) (width 0.2) (layer "F.Cu") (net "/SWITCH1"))
 (segment (start 145.5615 109.5) (end 131 109.5) (width 0.2) (layer "F.Cu") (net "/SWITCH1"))
 (segment (start 151.2065 106.395) (end 133 88.1885) (width 0.2) (layer "F.Cu") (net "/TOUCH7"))
 (segment (start 133 88.1885) (end 133 82.5) (width 0.2) (layer "F.Cu") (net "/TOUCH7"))
 (segment (start 139 76.5) (end 151 76.5) (width 0.2) (layer "F.Cu") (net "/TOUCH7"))
 (segment (start 133 82.5) (end 139 76.5) (width 0.2) (layer "F.Cu") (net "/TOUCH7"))
 (segment (start 151 76.5) (end 155.5 72) (width 0.2) (layer "F.Cu") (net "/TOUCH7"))
 (segment (start 153.7465 106.395) (end 153.7465 122.5535) (width 0.2) (layer "F.Cu") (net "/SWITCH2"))
 (segment (start 153.7465 122.5535) (end 151 125.3) (width 0.2) (layer "F.Cu") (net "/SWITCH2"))
 (segment (start 165.2991 109.761914) (end 165.2991 123.5991) (width 0.2) (layer "F.Cu") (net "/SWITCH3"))
 (segment (start 162.8525 107.315314) (end 165.2991 109.761914) (width 0.2) (layer "F.Cu") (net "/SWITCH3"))
 (segment (start 165.2991 123.5991) (end 167 125.3) (width 0.2) (layer "F.Cu") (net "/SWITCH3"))
 (segment (start 162.235082 105.341) (end 162.8525 105.958418) (width 0.2) (layer "F.Cu") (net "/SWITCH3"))
 (segment (start 162.8525 105.958418) (end 162.8525 107.315314) (width 0.2) (layer "F.Cu") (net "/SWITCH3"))
 (segment (start 157.3405 105.341) (end 162.235082 105.341) (width 0.2) (layer "F.Cu") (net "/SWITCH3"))
 (segment (start 156.2865 106.395) (end 157.3405 105.341) (width 0.2) (layer "F.Cu") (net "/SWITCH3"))
 (segment (start 151.2065 86.2935) (end 154.5 83) (width 0.2) (layer "F.Cu") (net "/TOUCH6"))
 (segment (start 151.2065 91.155) (end 151.2065 86.2935) (width 0.2) (layer "F.Cu") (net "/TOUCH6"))
 (segment (start 158.8265 91.155) (end 159.908645 90.072855) (width 0.2) (layer "F.Cu") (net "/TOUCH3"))
 (segment (start 159.908645 90.072855) (end 159.908645 82.408645) (width 0.2) (layer "F.Cu") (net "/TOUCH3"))
 (segment (start 159.908645 82.408645) (end 155.5 78) (width 0.2) (layer "F.Cu") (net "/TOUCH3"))
 (segment (start 152.2605 90.7395) (end 152.2605 92.2395) (width 0.2) (layer "F.Cu") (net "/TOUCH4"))
 (segment (start 152.899 90.101) (end 152.2605 90.7395) (width 0.2) (layer "F.Cu") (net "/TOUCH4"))
 (segment (start 156.2865 91.155) (end 155.2325 90.101) (width 0.2) (layer "F.Cu") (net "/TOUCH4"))
 (segment (start 142.5 83.497918) (end 142.5 78) (width 0.2) (layer "F.Cu") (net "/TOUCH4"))
 (segment (start 152 92.5) (end 150.628918 92.5) (width 0.2) (layer "F.Cu") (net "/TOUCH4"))
 (segment (start 152.2605 92.2395) (end 152 92.5) (width 0.2) (layer "F.Cu") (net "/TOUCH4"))
 (segment (start 155.2325 90.101) (end 152.899 90.101) (width 0.2) (layer "F.Cu") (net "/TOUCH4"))
 (segment (start 149.7205 90.718418) (end 142.5 83.497918) (width 0.2) (layer "F.Cu") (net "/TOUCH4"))
 (segment (start 150.628918 92.5) (end 149.7205 91.591582) (width 0.2) (layer "F.Cu") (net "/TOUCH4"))
 (segment (start 149.7205 91.591582) (end 149.7205 90.718418) (width 0.2) (layer "F.Cu") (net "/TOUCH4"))
 (segment (start 163.9065 91.155) (end 167.43285 87.62865) (width 0.2) (layer "F.Cu") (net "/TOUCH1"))
 (segment (start 167.43285 87.62865) (end 167.43285 80.828816) (width 0.2) (layer "F.Cu") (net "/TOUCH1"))
 (segment (start 152.91 76.59) (end 147.5 82) (width 0.2) (layer "F.Cu") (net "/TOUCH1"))
 (segment (start 167.43285 80.828816) (end 163.194034 76.59) (width 0.2) (layer "F.Cu") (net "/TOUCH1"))
 (segment (start 163.194034 76.59) (end 152.91 76.59) (width 0.2) (layer "F.Cu") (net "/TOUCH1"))
 (segment (start 161.3665 91.155) (end 161.3665 84.1335) (width 0.2) (layer "F.Cu") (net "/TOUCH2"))
 (segment (start 161.3665 84.1335) (end 163.5 82) (width 0.2) (layer "F.Cu") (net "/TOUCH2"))
 (segment (start 153.7465 91.155) (end 155.0915 92.5) (width 0.2) (layer "F.Cu") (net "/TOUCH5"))
 (segment (start 165 92.5) (end 168.5 89) (width 0.2) (layer "F.Cu") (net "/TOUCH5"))
 (segment (start 168.5 89) (end 168.5 78) (width 0.2) (layer "F.Cu") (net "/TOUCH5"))
 (segment (start 155.0915 92.5) (end 165 92.5) (width 0.2) (layer "F.Cu") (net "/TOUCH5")))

